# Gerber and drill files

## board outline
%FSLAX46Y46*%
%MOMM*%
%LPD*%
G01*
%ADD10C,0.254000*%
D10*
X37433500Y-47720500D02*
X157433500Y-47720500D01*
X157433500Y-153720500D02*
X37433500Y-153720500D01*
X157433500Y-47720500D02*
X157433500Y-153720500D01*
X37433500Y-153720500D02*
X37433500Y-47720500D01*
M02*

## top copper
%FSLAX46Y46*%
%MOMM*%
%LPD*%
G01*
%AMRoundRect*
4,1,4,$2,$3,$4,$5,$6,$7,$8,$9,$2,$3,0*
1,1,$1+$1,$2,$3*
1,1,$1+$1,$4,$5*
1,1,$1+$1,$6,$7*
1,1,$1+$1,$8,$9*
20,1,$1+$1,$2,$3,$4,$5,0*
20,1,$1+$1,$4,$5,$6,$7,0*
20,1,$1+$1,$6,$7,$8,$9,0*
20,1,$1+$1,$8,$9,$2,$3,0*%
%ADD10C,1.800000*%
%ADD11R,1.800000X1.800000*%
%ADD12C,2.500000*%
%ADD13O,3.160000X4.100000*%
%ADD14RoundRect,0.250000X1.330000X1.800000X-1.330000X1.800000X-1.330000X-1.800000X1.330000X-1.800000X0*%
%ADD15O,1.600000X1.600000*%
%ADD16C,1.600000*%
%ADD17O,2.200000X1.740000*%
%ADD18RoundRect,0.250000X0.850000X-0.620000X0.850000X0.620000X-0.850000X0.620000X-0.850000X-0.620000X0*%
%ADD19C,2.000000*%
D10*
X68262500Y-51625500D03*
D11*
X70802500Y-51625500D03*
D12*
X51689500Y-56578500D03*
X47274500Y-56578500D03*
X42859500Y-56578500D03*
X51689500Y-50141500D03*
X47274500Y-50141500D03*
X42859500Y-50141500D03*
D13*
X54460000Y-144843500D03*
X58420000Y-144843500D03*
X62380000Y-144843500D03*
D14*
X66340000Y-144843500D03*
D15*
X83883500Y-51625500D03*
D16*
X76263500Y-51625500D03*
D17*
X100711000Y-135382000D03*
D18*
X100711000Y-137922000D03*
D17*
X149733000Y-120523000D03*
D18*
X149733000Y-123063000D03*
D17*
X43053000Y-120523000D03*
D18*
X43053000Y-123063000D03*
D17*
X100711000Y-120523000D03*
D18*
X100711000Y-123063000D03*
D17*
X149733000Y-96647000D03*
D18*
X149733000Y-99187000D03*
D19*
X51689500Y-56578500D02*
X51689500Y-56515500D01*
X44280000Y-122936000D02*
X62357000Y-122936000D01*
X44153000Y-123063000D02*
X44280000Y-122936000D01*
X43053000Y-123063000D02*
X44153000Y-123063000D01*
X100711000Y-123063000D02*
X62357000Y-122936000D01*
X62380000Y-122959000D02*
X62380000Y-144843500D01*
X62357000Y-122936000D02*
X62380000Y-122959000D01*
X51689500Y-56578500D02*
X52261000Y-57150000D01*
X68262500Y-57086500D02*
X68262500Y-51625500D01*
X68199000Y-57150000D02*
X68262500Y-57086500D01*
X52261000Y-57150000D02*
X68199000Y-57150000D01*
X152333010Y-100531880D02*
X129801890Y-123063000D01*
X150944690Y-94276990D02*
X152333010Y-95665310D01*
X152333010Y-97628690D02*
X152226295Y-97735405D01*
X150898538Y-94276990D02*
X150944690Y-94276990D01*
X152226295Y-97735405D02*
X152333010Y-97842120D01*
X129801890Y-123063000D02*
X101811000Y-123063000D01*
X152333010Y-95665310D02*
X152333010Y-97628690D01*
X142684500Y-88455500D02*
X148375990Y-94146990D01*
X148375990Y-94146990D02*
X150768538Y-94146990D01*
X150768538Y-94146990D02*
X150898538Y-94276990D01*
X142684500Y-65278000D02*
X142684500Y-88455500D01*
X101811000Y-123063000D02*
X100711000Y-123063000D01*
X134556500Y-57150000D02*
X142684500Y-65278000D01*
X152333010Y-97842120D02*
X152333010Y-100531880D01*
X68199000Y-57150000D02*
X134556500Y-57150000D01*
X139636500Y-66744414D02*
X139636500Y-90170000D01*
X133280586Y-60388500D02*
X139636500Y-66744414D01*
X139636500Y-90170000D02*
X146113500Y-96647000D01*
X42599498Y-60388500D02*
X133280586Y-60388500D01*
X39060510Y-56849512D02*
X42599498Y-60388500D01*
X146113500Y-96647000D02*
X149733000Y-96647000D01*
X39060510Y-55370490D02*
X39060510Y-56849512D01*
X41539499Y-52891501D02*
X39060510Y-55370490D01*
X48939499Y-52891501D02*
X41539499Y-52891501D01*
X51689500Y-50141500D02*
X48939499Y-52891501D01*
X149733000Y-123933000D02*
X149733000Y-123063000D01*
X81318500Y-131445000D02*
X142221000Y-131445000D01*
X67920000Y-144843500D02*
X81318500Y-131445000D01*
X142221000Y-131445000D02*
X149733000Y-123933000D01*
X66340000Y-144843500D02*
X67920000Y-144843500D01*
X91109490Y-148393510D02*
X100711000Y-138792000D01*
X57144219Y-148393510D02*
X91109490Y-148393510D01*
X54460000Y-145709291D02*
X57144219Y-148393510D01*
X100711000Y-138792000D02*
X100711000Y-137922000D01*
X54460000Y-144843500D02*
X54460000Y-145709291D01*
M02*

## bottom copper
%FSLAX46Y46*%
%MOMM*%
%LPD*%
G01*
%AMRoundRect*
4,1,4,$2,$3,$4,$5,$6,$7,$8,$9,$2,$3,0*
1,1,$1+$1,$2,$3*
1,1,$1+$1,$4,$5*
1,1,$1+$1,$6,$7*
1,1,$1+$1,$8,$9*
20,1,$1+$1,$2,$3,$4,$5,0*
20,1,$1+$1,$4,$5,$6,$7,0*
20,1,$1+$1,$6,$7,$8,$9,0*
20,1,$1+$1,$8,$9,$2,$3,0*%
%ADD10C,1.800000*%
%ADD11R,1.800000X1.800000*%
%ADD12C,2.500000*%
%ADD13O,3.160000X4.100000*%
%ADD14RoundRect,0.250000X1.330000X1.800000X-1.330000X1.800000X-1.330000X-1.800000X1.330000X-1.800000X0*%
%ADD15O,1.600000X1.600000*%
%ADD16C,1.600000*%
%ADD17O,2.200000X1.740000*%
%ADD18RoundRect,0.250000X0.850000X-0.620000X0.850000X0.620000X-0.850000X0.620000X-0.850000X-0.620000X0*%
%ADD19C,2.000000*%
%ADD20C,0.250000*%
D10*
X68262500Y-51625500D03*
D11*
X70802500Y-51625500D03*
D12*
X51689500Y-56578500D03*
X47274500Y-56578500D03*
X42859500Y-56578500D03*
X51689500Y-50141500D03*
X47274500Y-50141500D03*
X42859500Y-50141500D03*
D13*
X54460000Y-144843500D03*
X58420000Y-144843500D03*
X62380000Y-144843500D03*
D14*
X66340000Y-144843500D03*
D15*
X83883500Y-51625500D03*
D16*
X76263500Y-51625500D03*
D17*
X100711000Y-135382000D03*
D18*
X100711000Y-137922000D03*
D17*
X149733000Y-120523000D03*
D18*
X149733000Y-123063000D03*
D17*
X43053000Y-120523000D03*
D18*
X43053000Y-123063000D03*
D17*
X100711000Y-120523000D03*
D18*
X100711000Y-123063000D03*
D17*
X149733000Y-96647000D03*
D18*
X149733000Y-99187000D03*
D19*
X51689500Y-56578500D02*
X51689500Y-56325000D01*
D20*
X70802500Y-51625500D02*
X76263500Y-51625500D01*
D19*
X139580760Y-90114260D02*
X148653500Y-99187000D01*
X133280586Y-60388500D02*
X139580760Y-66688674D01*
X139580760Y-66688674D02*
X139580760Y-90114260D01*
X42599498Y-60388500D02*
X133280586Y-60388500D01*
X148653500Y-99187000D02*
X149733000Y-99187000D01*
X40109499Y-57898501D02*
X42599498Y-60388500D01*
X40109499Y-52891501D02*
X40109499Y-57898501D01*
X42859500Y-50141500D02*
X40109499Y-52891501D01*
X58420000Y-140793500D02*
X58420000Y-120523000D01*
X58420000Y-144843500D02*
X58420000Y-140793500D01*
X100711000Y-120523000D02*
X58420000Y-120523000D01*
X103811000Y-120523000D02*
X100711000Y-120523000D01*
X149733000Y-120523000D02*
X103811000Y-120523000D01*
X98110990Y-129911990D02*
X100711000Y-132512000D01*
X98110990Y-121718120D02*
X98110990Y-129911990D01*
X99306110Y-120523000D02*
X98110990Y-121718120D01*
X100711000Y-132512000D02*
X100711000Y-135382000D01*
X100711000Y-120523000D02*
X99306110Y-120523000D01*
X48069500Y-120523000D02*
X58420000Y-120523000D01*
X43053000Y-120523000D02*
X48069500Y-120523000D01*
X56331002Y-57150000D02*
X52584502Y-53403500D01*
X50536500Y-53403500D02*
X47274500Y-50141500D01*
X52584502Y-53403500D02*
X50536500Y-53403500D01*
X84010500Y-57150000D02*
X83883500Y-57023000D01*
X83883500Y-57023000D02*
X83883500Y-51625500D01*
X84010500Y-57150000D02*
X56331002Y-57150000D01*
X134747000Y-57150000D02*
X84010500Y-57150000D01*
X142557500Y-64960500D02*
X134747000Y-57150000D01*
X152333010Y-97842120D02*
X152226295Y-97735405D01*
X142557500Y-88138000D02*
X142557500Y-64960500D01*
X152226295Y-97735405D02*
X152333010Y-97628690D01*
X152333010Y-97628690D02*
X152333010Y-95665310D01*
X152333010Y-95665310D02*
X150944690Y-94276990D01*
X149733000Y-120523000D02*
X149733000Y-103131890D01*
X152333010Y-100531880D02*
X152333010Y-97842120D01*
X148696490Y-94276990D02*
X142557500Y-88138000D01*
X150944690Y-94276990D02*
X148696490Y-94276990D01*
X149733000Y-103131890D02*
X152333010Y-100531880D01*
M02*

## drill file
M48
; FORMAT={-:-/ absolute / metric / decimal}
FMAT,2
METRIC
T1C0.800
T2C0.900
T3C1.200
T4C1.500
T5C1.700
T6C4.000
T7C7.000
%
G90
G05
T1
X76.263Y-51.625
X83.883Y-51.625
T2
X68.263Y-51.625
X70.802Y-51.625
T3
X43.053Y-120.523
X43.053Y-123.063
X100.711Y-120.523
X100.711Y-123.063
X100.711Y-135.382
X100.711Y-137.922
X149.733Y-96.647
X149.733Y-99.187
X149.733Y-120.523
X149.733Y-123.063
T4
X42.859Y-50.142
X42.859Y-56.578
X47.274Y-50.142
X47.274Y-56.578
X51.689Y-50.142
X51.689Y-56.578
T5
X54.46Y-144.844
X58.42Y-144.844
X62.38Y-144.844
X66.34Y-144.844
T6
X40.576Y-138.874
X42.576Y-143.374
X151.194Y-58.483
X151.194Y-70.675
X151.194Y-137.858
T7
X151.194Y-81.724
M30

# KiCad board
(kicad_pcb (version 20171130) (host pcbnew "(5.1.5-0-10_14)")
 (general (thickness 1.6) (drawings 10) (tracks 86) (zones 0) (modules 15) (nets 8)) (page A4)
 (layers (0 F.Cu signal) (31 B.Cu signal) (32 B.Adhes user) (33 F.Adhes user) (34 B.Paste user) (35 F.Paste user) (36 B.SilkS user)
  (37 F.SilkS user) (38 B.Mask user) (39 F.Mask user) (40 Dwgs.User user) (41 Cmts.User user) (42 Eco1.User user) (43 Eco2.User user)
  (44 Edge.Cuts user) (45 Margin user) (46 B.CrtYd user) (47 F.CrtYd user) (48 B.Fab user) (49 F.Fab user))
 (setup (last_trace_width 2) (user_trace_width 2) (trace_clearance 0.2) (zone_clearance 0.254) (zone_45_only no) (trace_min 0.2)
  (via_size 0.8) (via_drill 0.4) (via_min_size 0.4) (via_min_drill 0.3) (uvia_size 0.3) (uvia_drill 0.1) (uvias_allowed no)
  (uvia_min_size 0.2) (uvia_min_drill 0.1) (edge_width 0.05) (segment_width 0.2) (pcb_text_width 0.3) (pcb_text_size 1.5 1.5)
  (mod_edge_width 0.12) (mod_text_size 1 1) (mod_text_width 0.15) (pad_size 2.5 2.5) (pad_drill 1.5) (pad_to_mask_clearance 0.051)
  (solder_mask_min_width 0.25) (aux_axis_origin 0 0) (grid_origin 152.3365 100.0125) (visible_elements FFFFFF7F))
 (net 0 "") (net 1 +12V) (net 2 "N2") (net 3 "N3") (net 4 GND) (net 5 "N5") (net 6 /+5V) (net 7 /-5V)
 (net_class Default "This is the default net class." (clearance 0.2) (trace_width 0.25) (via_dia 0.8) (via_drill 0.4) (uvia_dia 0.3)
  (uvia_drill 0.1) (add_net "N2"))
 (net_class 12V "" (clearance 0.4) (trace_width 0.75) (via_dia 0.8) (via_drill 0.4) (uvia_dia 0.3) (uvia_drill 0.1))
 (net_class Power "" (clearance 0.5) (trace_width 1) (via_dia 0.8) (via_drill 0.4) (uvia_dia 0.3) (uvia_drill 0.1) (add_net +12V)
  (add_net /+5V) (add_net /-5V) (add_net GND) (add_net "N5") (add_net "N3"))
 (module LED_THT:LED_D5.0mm (layer F.Cu) (at 70.8025 51.6255 180)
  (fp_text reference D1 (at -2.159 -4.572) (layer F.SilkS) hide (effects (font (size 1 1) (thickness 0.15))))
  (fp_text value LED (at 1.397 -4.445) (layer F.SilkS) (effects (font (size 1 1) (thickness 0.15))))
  (pad 2 thru_hole circle (at 2.54 0 180) (size 1.8 1.8) (drill 0.9) (layers *.Cu *.Mask) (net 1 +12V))
  (pad 1 thru_hole rect (at 0 0 180) (size 1.8 1.8) (drill 0.9) (layers *.Cu *.Mask) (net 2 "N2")))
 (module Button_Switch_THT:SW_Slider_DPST (layer F.Cu) (at 47.3075 45.466)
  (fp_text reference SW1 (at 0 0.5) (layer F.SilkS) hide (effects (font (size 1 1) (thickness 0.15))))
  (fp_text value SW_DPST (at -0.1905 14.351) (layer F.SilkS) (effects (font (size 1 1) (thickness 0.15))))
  (pad 4 thru_hole circle (at 4.382 11.1125) (size 2.5 2.5) (drill 1.5) (layers *.Cu *.Paste *.Mask) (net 1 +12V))
  (pad 5 thru_hole circle (at -0.033 11.1125) (size 2.5 2.5) (drill 1.5) (layers *.Cu *.Paste *.Mask))
  (pad 6 thru_hole circle (at -4.448 11.1125) (size 2.5 2.5) (drill 1.5) (layers *.Cu *.Paste *.Mask))
  (pad 1 thru_hole circle (at 4.382 4.6755) (size 2.5 2.5) (drill 1.5) (layers *.Cu *.Paste *.Mask) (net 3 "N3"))
  (pad 2 thru_hole circle (at -0.033 4.6755) (size 2.5 2.5) (drill 1.5) (layers *.Cu *.Paste *.Mask) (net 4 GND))
  (pad 3 thru_hole circle (at -4.448 4.6755) (size 2.5 2.5) (drill 1.5) (layers *.Cu *.Paste *.Mask) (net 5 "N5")))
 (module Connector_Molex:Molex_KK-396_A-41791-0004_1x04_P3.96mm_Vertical (layer F.Cu) (at 66.34 144.8435 180)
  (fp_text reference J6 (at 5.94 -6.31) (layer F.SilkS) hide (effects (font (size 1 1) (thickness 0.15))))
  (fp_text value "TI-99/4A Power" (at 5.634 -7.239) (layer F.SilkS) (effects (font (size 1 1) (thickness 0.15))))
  (pad 4 thru_hole oval (at 11.88 0 180) (size 3.16 4.1) (drill 1.7) (layers *.Cu *.Mask) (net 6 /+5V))
  (pad 3 thru_hole oval (at 7.92 0 180) (size 3.16 4.1) (drill 1.7) (layers *.Cu *.Mask) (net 4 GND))
  (pad 2 thru_hole oval (at 3.96 0 180) (size 3.16 4.1) (drill 1.7) (layers *.Cu *.Mask) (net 1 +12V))
  (pad 1 thru_hole roundrect (at 0 0 180) (size 3.16 4.1) (drill 1.7) (layers *.Cu *.Mask) (roundrect_rratio 0.079114) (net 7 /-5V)))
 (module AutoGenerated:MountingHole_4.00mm (layer F.Cu) (at 42.5765 143.3745)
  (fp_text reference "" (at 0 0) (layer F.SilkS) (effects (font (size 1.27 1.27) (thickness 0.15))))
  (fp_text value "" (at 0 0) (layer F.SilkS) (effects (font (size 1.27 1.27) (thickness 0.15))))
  (pad "" np_thru_hole circle (at 0 0) (size 4 4) (drill 4) (layers *.Cu *.Mask)))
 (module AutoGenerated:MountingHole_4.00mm (layer F.Cu) (at 40.5765 138.8745)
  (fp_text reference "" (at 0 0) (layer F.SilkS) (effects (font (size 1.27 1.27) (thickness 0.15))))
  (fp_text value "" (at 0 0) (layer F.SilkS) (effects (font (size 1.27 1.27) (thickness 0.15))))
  (pad "" np_thru_hole circle (at 0 0) (size 4 4) (drill 4) (layers *.Cu *.Mask)))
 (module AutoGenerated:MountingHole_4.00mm (layer F.Cu) (at 151.1935 70.6755)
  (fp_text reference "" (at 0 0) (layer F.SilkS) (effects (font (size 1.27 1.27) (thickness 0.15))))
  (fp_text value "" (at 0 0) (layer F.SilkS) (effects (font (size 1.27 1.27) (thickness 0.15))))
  (pad "" np_thru_hole circle (at 0 0) (size 4 4) (drill 4) (layers *.Cu *.Mask)))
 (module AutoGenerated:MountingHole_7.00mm (layer F.Cu) (at 151.1935 81.7245)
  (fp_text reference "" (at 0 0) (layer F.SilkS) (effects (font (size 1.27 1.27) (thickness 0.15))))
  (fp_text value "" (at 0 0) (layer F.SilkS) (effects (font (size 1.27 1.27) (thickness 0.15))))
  (pad "" np_thru_hole circle (at 0 0) (size 7 7) (drill 7) (layers *.Cu *.Mask)))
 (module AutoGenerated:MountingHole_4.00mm (layer F.Cu) (at 151.1935 137.8585)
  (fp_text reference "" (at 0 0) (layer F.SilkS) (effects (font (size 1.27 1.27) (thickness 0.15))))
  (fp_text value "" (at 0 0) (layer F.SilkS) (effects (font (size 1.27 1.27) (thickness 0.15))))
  (pad "" np_thru_hole circle (at 0 0) (size 4 4) (drill 4) (layers *.Cu *.Mask)))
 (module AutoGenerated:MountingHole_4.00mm (layer F.Cu) (at 151.1935 58.4835)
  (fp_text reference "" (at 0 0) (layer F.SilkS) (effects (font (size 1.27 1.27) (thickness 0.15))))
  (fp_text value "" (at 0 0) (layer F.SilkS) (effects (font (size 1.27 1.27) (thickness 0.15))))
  (pad "" np_thru_hole circle (at 0 0) (size 4 4) (drill 4) (layers *.Cu *.Mask)))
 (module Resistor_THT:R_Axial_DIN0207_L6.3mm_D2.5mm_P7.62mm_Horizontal (layer F.Cu) (at 76.2635 51.6255)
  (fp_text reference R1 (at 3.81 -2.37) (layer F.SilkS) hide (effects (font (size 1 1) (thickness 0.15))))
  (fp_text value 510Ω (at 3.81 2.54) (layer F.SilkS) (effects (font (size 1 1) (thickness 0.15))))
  (pad 2 thru_hole oval (at 7.62 0) (size 1.6 1.6) (drill 0.8) (layers *.Cu *.Mask) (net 4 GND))
  (pad 1 thru_hole circle (at 0 0) (size 1.6 1.6) (drill 0.8) (layers *.Cu *.Mask) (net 2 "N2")))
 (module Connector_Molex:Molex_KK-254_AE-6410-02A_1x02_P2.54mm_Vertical (layer F.Cu) (at 100.711 137.922 90)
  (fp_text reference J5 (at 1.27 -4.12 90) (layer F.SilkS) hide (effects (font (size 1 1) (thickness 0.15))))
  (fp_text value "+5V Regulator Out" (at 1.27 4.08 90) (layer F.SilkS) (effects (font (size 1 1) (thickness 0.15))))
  (pad 2 thru_hole oval (at 2.54 0 90) (size 1.74 2.2) (drill 1.2) (layers *.Cu *.Mask) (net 4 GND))
  (pad 1 thru_hole roundrect (at 0 0 90) (size 1.74 2.2) (drill 1.2) (layers *.Cu *.Mask) (roundrect_rratio 0.143678) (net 6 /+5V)))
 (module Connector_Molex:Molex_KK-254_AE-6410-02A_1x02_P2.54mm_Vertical (layer F.Cu) (at 149.733 123.063 90)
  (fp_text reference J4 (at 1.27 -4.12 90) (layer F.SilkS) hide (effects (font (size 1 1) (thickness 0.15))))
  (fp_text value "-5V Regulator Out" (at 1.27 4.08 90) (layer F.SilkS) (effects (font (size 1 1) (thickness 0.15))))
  (pad 2 thru_hole oval (at 2.54 0 90) (size 1.74 2.2) (drill 1.2) (layers *.Cu *.Mask) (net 4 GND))
  (pad 1 thru_hole roundrect (at 0 0 90) (size 1.74 2.2) (drill 1.2) (layers *.Cu *.Mask) (roundrect_rratio 0.143678) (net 7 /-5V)))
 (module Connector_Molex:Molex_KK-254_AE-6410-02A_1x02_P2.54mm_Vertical (layer F.Cu) (at 43.053 123.063 90)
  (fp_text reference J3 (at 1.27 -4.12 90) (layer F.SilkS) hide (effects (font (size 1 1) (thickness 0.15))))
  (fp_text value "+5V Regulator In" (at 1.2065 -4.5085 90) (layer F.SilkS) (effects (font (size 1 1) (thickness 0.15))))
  (pad 2 thru_hole oval (at 2.54 0 90) (size 1.74 2.2) (drill 1.2) (layers *.Cu *.Mask) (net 4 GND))
  (pad 1 thru_hole roundrect (at 0 0 90) (size 1.74 2.2) (drill 1.2) (layers *.Cu *.Mask) (roundrect_rratio 0.143678) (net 1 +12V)))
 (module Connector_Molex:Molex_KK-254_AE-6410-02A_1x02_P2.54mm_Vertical (layer F.Cu) (at 100.711 123.063 90)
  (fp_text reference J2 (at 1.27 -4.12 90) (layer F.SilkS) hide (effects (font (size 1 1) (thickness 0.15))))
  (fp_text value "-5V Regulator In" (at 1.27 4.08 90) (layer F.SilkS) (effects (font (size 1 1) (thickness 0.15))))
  (pad 2 thru_hole oval (at 2.54 0 90) (size 1.74 2.2) (drill 1.2) (layers *.Cu *.Mask) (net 4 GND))
  (pad 1 thru_hole roundrect (at 0 0 90) (size 1.74 2.2) (drill 1.2) (layers *.Cu *.Mask) (roundrect_rratio 0.143678) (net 1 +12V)))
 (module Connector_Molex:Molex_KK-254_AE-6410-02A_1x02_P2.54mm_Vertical (layer F.Cu) (at 149.733 99.187 90)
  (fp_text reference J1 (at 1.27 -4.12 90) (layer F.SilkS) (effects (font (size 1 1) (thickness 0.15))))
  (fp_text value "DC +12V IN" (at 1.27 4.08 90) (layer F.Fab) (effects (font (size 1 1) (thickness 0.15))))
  (pad 2 thru_hole oval (at 2.54 0 90) (size 1.74 2.2) (drill 1.2) (layers *.Cu *.Mask) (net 3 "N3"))
  (pad 1 thru_hole roundrect (at 0 0 90) (size 1.74 2.2) (drill 1.2) (layers *.Cu *.Mask) (roundrect_rratio 0.143678) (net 5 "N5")))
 (gr_line (start 37.4335 47.7205) (end 157.4335 47.7205) (layer Edge.Cuts) (width 0.254))
 (gr_line (start 157.4335 153.7205) (end 37.4335 153.7205) (layer Edge.Cuts) (width 0.254))
 (gr_line (start 157.4335 47.7205) (end 157.4335 153.7205) (layer Edge.Cuts) (width 0.254))
 (gr_line (start 37.4335 153.7205) (end 37.4335 47.7205) (layer Edge.Cuts) (width 0.254))
 (segment (start 51.6895 56.5785) (end 51.6895 56.325) (width 2) (layer B.Cu) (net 1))
 (segment (start 51.6895 56.5785) (end 51.6895 56.5155) (width 2) (layer F.Cu) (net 1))
 (segment (start 44.28 122.936) (end 62.357 122.936) (width 2) (layer F.Cu) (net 1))
 (segment (start 44.153 123.063) (end 44.28 122.936) (width 2) (layer F.Cu) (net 1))
 (segment (start 43.053 123.063) (end 44.153 123.063) (width 2) (layer F.Cu) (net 1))
 (segment (start 100.711 123.063) (end 62.357 122.936) (width 2) (layer F.Cu) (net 1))
 (segment (start 62.38 122.959) (end 62.38 144.8435) (width 2) (layer F.Cu) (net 1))
 (segment (start 62.357 122.936) (end 62.38 122.959) (width 2) (layer F.Cu) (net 1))
 (segment (start 51.6895 56.5785) (end 52.261 57.15) (width 2) (layer F.Cu) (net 1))
 (segment (start 68.2625 57.0865) (end 68.2625 51.6255) (width 2) (layer F.Cu) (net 1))
 (segment (start 68.199 57.15) (end 68.2625 57.0865) (width 2) (layer F.Cu) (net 1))
 (segment (start 52.261 57.15) (end 68.199 57.15) (width 2) (layer F.Cu) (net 1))
 (segment (start 152.33301 100.53188) (end 129.80189 123.063) (width 2) (layer F.Cu) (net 1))
 (segment (start 150.94469 94.27699) (end 152.33301 95.66531) (width 2) (layer F.Cu) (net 1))
 (segment (start 152.33301 97.62869) (end 152.226295 97.735405) (width 2) (layer F.Cu) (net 1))
 (segment (start 150.898538 94.27699) (end 150.94469 94.27699) (width 2) (layer F.Cu) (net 1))
 (segment (start 152.226295 97.735405) (end 152.33301 97.84212) (width 2) (layer F.Cu) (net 1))
 (segment (start 129.80189 123.063) (end 101.811 123.063) (width 2) (layer F.Cu) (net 1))
 (segment (start 152.33301 95.66531) (end 152.33301 97.62869) (width 2) (layer F.Cu) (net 1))
 (segment (start 142.6845 88.4555) (end 148.37599 94.14699) (width 2) (layer F.Cu) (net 1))
 (segment (start 148.37599 94.14699) (end 150.768538 94.14699) (width 2) (layer F.Cu) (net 1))
 (segment (start 150.768538 94.14699) (end 150.898538 94.27699) (width 2) (layer F.Cu) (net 1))
 (segment (start 142.6845 65.278) (end 142.6845 88.4555) (width 2) (layer F.Cu) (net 1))
 (segment (start 101.811 123.063) (end 100.711 123.063) (width 2) (layer F.Cu) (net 1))
 (segment (start 134.5565 57.15) (end 142.6845 65.278) (width 2) (layer F.Cu) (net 1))
 (segment (start 152.33301 97.84212) (end 152.33301 100.53188) (width 2) (layer F.Cu) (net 1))
 (segment (start 68.199 57.15) (end 134.5565 57.15) (width 2) (layer F.Cu) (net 1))
 (segment (start 70.8025 51.6255) (end 76.2635 51.6255) (width 0.25) (layer B.Cu) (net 2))
 (segment (start 139.6365 66.744414) (end 139.6365 90.17) (width 2) (layer F.Cu) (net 3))
 (segment (start 133.280586 60.3885) (end 139.6365 66.744414) (width 2) (layer F.Cu) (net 3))
 (segment (start 139.6365 90.17) (end 146.1135 96.647) (width 2) (layer F.Cu) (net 3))
 (segment (start 42.599498 60.3885) (end 133.280586 60.3885) (width 2) (layer F.Cu) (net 3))
 (segment (start 39.06051 56.849512) (end 42.599498 60.3885) (width 2) (layer F.Cu) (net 3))
 (segment (start 146.1135 96.647) (end 149.733 96.647) (width 2) (layer F.Cu) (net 3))
 (segment (start 39.06051 55.37049) (end 39.06051 56.849512) (width 2) (layer F.Cu) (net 3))
 (segment (start 41.539499 52.891501) (end 39.06051 55.37049) (width 2) (layer F.Cu) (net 3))
 (segment (start 48.939499 52.891501) (end 41.539499 52.891501) (width 2) (layer F.Cu) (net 3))
 (segment (start 51.6895 50.1415) (end 48.939499 52.891501) (width 2) (layer F.Cu) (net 3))
 (segment (start 139.58076 90.11426) (end 148.6535 99.187) (width 2) (layer B.Cu) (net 5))
 (segment (start 133.280586 60.3885) (end 139.58076 66.688674) (width 2) (layer B.Cu) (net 5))
 (segment (start 139.58076 66.688674) (end 139.58076 90.11426) (width 2) (layer B.Cu) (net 5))
 (segment (start 42.599498 60.3885) (end 133.280586 60.3885) (width 2) (layer B.Cu) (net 5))
 (segment (start 148.6535 99.187) (end 149.733 99.187) (width 2) (layer B.Cu) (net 5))
 (segment (start 40.109499 57.898501) (end 42.599498 60.3885) (width 2) (layer B.Cu) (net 5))
 (segment (start 40.109499 52.891501) (end 40.109499 57.898501) (width 2) (layer B.Cu) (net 5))
 (segment (start 42.8595 50.1415) (end 40.109499 52.891501) (width 2) (layer B.Cu) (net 5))
 (segment (start 58.42 140.7935) (end 58.42 120.523) (width 2) (layer B.Cu) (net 4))
 (segment (start 58.42 144.8435) (end 58.42 140.7935) (width 2) (layer B.Cu) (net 4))
 (segment (start 100.711 120.523) (end 58.42 120.523) (width 2) (layer B.Cu) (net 4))
 (segment (start 103.811 120.523) (end 100.711 120.523) (width 2) (layer B.Cu) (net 4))
 (segment (start 149.733 120.523) (end 103.811 120.523) (width 2) (layer B.Cu) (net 4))
 (segment (start 98.11099 129.91199) (end 100.711 132.512) (width 2) (layer B.Cu) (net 4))
 (segment (start 98.11099 121.71812) (end 98.11099 129.91199) (width 2) (layer B.Cu) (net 4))
 (segment (start 99.30611 120.523) (end 98.11099 121.71812) (width 2) (layer B.Cu) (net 4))
 (segment (start 100.711 132.512) (end 100.711 135.382) (width 2) (layer B.Cu) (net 4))
 (segment (start 100.711 120.523) (end 99.30611 120.523) (width 2) (layer B.Cu) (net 4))
 (segment (start 48.0695 120.523) (end 58.42 120.523) (width 2) (layer B.Cu) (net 4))
 (segment (start 43.053 120.523) (end 48.0695 120.523) (width 2) (layer B.Cu) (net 4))
 (segment (start 56.331002 57.15) (end 52.584502 53.4035) (width 2) (layer B.Cu) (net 4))
 (segment (start 50.5365 53.4035) (end 47.2745 50.1415) (width 2) (layer B.Cu) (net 4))
 (segment (start 52.584502 53.4035) (end 50.5365 53.4035) (width 2) (layer B.Cu) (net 4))
 (segment (start 84.0105 57.15) (end 83.8835 57.023) (width 2) (layer B.Cu) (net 4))
 (segment (start 83.8835 57.023) (end 83.8835 51.6255) (width 2) (layer B.Cu) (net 4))
 (segment (start 84.0105 57.15) (end 56.331002 57.15) (width 2) (layer B.Cu) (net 4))
 (segment (start 134.747 57.15) (end 84.0105 57.15) (width 2) (layer B.Cu) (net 4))
 (segment (start 142.5575 64.9605) (end 134.747 57.15) (width 2) (layer B.Cu) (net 4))
 (segment (start 152.33301 97.84212) (end 152.226295 97.735405) (width 2) (layer B.Cu) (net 4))
 (segment (start 142.5575 88.138) (end 142.5575 64.9605) (width 2) (layer B.Cu) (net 4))
 (segment (start 152.226295 97.735405) (end 152.33301 97.62869) (width 2) (layer B.Cu) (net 4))
 (segment (start 152.33301 97.62869) (end 152.33301 95.66531) (width 2) (layer B.Cu) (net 4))
 (segment (start 152.33301 95.66531) (end 150.94469 94.27699) (width 2) (layer B.Cu) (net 4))
 (segment (start 149.733 120.523) (end 149.733 103.13189) (width 2) (layer B.Cu) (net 4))
 (segment (start 152.33301 100.53188) (end 152.33301 97.84212) (width 2) (layer B.Cu) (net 4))
 (segment (start 148.69649 94.27699) (end 142.5575 88.138) (width 2) (layer B.Cu) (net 4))
 (segment (start 150.94469 94.27699) (end 148.69649 94.27699) (width 2) (layer B.Cu) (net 4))
 (segment (start 149.733 103.13189) (end 152.33301 100.53188) (width 2) (layer B.Cu) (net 4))
 (segment (start 149.733 123.933) (end 149.733 123.063) (width 2) (layer F.Cu) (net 7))
 (segment (start 81.3185 131.445) (end 142.221 131.445) (width 2) (layer F.Cu) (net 7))
 (segment (start 67.92 144.8435) (end 81.3185 131.445) (width 2) (layer F.Cu) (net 7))
 (segment (start 142.221 131.445) (end 149.733 123.933) (width 2) (layer F.Cu) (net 7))
 (segment (start 66.34 144.8435) (end 67.92 144.8435) (width 2) (layer F.Cu) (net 7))
 (segment (start 91.10949 148.39351) (end 100.711 138.792) (width 2) (layer F.Cu) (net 6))
 (segment (start 57.144219 148.39351) (end 91.10949 148.39351) (width 2) (layer F.Cu) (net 6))
 (segment (start 54.46 145.709291) (end 57.144219 148.39351) (width 2) (layer F.Cu) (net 6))
 (segment (start 100.711 138.792) (end 100.711 137.922) (width 2) (layer F.Cu) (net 6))
 (segment (start 54.46 144.8435) (end 54.46 145.709291) (width 2) (layer F.Cu) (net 6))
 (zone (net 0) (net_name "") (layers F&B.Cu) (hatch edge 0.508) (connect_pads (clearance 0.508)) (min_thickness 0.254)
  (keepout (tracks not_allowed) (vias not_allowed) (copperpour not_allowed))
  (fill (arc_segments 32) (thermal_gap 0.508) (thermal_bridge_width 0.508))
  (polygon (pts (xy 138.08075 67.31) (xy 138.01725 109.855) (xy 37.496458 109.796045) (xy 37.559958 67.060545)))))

